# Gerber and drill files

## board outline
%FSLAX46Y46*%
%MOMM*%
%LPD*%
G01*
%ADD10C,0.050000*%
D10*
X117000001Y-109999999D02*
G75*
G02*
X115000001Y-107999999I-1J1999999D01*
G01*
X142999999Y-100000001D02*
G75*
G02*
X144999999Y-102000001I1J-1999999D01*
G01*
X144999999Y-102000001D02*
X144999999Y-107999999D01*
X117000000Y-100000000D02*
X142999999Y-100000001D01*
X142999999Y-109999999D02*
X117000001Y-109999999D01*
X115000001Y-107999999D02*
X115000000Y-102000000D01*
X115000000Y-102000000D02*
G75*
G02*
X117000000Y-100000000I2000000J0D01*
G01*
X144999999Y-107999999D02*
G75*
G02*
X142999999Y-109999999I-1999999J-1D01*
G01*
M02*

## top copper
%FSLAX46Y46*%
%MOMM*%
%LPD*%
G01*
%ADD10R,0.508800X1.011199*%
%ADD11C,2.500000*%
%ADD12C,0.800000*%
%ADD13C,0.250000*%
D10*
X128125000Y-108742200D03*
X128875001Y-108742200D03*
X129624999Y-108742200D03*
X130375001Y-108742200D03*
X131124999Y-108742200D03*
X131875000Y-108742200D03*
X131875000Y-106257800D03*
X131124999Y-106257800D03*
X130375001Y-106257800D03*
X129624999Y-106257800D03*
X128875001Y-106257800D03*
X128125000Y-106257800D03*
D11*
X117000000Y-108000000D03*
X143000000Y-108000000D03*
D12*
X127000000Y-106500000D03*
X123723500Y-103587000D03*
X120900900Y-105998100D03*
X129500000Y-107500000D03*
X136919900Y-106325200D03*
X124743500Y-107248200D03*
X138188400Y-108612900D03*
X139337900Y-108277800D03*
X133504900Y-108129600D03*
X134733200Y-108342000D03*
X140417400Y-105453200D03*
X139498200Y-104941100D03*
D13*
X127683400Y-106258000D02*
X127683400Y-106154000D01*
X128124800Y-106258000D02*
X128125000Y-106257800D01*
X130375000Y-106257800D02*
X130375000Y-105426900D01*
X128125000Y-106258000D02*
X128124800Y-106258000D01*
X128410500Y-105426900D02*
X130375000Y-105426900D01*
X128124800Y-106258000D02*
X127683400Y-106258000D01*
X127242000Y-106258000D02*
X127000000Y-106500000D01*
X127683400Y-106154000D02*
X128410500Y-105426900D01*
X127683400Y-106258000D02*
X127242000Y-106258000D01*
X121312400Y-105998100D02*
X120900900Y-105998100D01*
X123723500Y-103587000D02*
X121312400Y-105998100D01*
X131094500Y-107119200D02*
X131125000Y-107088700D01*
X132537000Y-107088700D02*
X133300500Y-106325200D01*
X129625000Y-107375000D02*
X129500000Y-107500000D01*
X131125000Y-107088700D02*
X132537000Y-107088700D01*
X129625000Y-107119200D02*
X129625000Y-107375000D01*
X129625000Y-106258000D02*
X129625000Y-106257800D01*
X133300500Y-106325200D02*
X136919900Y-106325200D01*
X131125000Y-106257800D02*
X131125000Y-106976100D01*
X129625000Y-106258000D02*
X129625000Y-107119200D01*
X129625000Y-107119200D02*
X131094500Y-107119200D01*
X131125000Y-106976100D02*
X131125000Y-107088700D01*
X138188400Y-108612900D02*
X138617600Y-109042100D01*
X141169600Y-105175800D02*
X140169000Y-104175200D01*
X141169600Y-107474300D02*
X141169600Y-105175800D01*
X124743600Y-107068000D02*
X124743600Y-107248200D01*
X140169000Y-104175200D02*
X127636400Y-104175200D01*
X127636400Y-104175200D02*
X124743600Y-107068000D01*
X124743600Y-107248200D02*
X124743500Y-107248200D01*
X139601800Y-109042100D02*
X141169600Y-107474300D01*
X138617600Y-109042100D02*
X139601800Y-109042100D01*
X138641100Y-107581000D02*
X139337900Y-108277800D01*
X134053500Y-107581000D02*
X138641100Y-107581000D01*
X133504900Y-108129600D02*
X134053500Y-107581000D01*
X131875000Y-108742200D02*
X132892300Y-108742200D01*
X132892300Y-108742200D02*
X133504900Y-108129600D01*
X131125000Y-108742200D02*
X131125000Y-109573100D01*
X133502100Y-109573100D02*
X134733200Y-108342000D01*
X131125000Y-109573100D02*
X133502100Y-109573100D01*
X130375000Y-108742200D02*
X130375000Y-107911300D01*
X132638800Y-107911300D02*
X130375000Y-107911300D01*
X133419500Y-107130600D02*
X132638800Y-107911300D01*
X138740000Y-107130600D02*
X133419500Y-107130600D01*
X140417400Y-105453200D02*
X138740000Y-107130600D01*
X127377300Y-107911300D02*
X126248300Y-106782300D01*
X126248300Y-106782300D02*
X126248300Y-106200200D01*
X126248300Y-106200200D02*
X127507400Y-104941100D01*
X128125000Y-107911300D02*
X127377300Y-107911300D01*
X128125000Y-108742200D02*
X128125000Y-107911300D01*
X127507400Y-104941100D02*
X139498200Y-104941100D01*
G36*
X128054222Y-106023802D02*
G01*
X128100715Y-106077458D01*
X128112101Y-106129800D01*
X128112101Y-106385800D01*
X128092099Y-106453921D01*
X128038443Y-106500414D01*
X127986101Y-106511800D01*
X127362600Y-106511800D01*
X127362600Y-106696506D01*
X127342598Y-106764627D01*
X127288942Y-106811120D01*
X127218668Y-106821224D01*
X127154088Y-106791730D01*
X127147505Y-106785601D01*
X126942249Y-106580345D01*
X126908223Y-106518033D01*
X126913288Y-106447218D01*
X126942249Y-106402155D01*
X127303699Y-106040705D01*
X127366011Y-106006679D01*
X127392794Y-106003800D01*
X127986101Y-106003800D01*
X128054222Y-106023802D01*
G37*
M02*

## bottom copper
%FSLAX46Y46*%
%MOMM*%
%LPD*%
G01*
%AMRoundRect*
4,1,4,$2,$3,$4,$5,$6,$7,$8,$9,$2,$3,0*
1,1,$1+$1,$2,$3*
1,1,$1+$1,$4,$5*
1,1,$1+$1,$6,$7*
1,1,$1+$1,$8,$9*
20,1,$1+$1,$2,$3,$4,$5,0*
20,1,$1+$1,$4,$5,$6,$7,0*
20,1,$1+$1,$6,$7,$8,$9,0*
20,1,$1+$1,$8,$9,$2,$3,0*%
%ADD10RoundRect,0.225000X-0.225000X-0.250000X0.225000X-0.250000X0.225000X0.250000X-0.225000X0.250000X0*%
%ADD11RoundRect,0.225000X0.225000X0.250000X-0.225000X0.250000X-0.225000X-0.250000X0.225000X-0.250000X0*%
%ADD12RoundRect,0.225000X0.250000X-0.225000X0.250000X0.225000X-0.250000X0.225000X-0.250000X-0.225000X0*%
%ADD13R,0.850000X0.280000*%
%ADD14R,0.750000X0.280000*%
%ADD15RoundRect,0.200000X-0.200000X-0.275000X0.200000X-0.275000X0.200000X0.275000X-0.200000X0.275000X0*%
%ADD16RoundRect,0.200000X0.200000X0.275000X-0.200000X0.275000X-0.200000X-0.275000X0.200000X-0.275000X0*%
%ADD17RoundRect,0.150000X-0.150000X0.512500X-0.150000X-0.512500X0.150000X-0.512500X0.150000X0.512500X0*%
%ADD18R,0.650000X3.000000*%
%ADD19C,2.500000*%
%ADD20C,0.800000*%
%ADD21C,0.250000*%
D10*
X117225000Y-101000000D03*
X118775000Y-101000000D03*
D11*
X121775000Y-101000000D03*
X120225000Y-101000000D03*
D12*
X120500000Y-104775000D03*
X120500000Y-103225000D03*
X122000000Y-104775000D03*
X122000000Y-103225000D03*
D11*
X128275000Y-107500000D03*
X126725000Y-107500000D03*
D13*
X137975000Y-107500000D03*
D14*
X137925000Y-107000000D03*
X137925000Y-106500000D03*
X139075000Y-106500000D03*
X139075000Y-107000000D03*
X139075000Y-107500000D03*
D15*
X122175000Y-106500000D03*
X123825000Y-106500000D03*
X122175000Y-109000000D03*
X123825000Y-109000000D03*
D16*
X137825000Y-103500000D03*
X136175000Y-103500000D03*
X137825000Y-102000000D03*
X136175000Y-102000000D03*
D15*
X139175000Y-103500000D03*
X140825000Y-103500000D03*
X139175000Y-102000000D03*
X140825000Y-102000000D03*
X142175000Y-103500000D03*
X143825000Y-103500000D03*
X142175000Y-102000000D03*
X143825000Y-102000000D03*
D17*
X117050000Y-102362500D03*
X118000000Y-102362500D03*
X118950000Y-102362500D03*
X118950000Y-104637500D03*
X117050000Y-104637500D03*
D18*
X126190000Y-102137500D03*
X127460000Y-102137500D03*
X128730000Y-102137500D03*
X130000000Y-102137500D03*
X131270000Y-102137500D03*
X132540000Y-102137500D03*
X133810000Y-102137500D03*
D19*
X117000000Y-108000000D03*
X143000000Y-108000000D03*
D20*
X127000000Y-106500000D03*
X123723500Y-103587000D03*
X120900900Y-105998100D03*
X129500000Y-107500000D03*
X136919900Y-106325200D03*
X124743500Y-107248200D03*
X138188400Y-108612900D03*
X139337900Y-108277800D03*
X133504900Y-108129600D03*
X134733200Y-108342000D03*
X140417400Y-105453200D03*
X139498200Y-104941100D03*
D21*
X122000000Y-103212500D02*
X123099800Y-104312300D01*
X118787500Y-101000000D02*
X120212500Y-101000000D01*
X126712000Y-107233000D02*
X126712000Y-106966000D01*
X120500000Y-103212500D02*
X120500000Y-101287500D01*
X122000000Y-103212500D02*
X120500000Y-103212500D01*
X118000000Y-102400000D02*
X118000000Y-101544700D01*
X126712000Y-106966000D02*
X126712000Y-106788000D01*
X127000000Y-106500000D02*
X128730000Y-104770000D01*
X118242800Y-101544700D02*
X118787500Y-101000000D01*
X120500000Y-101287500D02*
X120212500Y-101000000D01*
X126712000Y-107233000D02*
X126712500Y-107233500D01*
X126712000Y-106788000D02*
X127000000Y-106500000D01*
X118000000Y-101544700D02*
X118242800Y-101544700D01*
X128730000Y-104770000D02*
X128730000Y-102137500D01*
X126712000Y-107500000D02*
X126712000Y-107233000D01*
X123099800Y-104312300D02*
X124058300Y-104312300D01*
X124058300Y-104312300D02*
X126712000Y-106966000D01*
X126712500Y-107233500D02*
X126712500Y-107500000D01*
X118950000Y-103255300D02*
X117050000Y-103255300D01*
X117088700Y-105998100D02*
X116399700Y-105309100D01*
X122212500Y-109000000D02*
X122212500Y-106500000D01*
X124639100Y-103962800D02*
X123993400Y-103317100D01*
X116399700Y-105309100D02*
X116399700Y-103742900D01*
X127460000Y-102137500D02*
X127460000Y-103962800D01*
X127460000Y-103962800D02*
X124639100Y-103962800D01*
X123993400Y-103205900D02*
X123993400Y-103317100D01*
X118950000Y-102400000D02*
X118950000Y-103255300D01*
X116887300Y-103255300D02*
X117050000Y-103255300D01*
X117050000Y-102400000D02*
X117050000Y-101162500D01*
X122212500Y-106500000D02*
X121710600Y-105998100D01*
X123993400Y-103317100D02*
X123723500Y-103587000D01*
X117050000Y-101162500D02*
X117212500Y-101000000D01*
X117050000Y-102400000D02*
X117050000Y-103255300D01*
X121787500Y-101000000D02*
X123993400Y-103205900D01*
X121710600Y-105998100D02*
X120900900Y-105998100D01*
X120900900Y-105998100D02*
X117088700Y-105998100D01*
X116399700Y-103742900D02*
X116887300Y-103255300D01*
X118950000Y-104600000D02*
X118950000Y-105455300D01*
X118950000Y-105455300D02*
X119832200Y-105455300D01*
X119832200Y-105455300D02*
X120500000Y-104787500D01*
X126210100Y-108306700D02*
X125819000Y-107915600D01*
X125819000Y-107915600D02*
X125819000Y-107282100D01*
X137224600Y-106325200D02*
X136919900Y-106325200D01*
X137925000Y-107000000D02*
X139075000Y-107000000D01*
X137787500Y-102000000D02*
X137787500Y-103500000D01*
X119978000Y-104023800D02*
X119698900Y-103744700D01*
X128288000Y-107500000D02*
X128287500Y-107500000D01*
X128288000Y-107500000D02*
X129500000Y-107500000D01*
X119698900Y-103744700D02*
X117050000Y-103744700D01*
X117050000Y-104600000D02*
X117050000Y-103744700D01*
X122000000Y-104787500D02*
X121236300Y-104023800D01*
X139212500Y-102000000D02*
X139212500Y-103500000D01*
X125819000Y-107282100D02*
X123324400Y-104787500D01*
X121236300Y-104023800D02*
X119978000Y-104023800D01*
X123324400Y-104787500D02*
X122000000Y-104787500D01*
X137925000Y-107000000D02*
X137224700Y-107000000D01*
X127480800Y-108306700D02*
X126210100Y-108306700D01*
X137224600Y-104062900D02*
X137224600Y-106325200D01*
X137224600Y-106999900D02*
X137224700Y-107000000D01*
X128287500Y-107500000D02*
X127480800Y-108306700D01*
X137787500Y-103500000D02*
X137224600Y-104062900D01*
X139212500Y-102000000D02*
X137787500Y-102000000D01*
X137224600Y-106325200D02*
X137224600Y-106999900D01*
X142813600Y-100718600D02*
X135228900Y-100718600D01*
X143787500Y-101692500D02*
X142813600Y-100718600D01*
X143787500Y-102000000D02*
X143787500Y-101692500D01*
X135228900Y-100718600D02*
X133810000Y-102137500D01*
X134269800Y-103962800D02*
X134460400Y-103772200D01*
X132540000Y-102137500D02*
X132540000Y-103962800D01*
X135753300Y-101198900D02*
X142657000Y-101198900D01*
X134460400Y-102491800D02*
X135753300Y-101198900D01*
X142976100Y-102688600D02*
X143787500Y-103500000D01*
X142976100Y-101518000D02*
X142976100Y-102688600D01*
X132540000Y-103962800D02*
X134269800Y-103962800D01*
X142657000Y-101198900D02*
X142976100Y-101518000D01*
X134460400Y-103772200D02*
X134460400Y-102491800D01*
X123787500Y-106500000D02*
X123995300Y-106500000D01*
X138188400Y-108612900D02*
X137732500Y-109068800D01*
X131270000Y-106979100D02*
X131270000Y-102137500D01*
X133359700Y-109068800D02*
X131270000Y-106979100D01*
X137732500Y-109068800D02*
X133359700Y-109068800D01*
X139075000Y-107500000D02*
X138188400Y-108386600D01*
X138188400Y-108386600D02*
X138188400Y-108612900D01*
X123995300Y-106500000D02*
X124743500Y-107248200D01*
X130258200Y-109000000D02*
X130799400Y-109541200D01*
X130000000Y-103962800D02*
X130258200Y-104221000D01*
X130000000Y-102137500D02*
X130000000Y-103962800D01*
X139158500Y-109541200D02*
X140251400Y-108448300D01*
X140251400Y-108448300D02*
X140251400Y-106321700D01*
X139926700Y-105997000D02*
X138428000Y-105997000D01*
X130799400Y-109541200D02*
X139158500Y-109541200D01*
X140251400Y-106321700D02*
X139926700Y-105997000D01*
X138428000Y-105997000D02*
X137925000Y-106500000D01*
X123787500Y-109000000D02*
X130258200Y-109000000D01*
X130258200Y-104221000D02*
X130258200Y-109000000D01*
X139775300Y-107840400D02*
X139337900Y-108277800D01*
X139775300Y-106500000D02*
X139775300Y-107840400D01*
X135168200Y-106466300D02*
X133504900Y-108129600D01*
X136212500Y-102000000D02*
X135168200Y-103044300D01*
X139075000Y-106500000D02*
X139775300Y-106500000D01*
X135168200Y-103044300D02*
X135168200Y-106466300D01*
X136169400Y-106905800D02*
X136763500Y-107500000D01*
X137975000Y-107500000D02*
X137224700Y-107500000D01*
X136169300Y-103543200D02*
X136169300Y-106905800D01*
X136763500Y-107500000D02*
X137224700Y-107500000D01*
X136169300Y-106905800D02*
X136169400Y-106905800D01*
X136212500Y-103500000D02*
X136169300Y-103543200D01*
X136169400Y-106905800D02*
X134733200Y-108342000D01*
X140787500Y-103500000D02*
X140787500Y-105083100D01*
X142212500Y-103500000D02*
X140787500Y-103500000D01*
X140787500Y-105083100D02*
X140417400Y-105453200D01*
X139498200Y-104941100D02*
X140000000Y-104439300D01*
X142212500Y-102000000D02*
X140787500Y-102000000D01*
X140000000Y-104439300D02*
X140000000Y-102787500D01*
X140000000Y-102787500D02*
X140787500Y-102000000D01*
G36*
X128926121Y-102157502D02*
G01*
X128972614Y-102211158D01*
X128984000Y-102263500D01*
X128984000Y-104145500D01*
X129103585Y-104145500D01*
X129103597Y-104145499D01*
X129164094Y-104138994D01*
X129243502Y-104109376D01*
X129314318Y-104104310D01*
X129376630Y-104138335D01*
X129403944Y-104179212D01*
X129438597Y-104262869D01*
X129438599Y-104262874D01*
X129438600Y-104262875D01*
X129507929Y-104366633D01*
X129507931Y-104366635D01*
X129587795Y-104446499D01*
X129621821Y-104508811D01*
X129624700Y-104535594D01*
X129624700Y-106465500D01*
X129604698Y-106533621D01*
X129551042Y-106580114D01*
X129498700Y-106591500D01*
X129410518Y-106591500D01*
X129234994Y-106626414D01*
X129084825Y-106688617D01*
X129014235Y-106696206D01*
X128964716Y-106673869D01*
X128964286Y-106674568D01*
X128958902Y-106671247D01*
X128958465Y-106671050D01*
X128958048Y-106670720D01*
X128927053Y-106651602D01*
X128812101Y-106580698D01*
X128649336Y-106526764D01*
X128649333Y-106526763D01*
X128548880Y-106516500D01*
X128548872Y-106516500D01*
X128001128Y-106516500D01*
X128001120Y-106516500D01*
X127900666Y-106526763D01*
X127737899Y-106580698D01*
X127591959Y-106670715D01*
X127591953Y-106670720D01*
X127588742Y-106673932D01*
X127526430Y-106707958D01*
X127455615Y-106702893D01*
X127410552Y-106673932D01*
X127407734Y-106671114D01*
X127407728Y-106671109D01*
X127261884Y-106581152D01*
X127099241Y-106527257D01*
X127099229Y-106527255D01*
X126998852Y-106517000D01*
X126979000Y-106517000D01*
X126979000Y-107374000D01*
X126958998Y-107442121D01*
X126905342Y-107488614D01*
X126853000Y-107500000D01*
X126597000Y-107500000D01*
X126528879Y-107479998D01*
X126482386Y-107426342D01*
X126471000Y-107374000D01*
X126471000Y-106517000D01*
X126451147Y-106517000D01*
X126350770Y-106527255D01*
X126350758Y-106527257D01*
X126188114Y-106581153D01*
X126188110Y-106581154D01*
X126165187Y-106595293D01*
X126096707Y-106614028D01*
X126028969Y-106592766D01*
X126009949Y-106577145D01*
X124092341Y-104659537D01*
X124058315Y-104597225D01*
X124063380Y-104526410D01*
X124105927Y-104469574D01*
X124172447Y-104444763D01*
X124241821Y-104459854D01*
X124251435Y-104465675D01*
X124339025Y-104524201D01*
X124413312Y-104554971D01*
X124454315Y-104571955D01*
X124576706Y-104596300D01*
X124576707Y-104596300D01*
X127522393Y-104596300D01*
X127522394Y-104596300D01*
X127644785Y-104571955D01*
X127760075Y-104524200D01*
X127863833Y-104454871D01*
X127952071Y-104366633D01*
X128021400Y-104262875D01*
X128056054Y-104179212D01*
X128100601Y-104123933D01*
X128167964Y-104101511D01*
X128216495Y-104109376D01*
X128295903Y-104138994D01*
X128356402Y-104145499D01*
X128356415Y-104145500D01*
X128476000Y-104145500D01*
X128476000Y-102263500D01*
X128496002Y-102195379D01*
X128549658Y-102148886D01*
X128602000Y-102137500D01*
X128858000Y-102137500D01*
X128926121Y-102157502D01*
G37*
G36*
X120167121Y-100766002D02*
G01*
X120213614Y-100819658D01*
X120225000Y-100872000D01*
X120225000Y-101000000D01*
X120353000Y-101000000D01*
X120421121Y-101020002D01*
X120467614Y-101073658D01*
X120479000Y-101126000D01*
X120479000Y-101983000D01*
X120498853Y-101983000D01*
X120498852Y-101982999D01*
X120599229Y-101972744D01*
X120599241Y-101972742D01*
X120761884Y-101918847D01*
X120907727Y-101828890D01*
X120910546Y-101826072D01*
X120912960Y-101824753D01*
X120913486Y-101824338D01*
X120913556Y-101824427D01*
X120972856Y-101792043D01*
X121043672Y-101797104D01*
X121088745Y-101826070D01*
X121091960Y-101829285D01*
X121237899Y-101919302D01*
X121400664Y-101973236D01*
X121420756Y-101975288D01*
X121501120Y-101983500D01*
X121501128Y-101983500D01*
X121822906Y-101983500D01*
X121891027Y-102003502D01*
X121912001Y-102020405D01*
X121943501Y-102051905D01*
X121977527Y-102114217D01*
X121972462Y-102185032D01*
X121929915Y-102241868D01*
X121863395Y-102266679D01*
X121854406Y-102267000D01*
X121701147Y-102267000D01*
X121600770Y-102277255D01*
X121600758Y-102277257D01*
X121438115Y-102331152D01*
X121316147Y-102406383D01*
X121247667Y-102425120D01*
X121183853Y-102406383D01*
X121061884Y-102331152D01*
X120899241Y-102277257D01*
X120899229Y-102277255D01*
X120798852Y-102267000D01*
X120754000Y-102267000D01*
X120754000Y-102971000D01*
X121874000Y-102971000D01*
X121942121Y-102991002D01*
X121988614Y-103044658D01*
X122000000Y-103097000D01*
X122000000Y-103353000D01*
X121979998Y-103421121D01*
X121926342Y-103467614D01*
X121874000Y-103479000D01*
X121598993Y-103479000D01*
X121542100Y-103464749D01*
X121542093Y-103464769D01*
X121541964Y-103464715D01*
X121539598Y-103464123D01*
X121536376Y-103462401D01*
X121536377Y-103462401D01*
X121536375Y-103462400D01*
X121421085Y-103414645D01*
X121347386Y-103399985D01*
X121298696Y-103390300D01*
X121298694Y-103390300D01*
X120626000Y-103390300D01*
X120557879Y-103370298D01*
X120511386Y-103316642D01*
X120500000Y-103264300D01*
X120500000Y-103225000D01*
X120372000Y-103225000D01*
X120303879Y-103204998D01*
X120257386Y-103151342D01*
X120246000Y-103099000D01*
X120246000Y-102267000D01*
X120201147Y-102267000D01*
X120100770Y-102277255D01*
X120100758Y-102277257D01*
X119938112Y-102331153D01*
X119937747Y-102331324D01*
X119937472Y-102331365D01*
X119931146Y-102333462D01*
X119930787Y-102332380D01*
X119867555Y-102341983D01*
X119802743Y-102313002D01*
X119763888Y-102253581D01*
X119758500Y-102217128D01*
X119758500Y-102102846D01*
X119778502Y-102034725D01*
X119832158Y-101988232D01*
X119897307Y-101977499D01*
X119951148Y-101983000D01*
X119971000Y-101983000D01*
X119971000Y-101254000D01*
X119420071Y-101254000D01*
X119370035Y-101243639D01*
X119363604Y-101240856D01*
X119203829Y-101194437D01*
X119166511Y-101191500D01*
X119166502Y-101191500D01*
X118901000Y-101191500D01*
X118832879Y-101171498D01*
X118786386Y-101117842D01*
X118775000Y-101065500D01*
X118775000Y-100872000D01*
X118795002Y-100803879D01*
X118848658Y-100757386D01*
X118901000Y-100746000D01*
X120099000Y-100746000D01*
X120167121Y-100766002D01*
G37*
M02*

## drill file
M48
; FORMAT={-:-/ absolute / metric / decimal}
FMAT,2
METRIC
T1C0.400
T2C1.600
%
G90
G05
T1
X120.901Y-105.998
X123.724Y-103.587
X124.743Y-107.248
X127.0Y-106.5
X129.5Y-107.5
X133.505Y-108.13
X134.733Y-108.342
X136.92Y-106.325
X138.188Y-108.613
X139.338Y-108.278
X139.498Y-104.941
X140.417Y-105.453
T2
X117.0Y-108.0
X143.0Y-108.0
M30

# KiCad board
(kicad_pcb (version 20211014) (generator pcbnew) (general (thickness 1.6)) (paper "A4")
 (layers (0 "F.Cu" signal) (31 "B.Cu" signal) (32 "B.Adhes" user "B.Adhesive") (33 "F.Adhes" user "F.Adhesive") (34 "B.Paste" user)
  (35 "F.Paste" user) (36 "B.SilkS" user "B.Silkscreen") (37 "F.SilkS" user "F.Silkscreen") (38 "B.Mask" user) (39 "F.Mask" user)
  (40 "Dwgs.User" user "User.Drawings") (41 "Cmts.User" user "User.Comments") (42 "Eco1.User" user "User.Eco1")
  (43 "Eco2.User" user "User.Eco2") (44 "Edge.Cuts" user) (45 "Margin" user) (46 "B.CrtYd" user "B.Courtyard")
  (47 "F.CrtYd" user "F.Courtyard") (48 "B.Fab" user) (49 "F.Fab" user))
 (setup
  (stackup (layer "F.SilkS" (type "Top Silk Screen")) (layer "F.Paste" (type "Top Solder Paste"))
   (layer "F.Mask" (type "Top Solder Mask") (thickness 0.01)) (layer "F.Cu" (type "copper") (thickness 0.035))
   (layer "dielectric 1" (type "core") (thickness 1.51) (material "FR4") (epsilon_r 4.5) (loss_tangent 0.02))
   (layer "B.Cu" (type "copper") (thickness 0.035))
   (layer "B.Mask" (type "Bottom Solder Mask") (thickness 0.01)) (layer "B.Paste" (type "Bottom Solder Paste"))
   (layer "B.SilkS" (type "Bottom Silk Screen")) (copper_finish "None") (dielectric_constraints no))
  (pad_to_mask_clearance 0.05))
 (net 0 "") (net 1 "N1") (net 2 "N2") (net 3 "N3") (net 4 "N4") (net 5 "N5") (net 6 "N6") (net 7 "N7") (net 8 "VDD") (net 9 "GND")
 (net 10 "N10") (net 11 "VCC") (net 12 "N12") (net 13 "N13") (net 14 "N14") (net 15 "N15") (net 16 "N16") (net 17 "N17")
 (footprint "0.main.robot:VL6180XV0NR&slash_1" (layer "F.Cu") (at 130 107.5 90)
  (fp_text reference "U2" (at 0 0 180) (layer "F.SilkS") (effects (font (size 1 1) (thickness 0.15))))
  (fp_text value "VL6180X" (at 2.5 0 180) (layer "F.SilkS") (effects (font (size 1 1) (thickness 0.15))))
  (pad "1" smd rect (at -1.2422 -1.875 90) (size 1.011199 0.5088) (layers "F.Cu" "F.Paste" "F.Mask") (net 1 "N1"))
  (pad "2" smd rect (at -1.2422 -1.124999 90) (size 1.011199 0.5088) (layers "F.Cu" "F.Paste" "F.Mask") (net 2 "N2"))
  (pad "3" smd rect (at -1.2422 -0.375001 90) (size 1.011199 0.5088) (layers "F.Cu" "F.Paste" "F.Mask") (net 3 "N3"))
  (pad "4" smd rect (at -1.2422 0.375001 90) (size 1.011199 0.5088) (layers "F.Cu" "F.Paste" "F.Mask") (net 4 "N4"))
  (pad "5" smd rect (at -1.2422 1.124999 90) (size 1.011199 0.5088) (layers "F.Cu" "F.Paste" "F.Mask") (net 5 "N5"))
  (pad "6" smd rect (at -1.2422 1.875 90) (size 1.011199 0.5088) (layers "F.Cu" "F.Paste" "F.Mask") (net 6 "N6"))
  (pad "7" smd rect (at 1.2422 1.875 90) (size 1.011199 0.5088) (layers "F.Cu" "F.Paste" "F.Mask") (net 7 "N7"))
  (pad "8" smd rect (at 1.2422 1.124999 90) (size 1.011199 0.5088) (layers "F.Cu" "F.Paste" "F.Mask") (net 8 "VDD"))
  (pad "9" smd rect (at 1.2422 0.375001 90) (size 1.011199 0.5088) (layers "F.Cu" "F.Paste" "F.Mask") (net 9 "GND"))
  (pad "10" smd rect (at 1.2422 -0.375001 90) (size 1.011199 0.5088) (layers "F.Cu" "F.Paste" "F.Mask") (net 8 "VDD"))
  (pad "11" smd rect (at 1.2422 -1.124999 90) (size 1.011199 0.5088) (layers "F.Cu" "F.Paste" "F.Mask") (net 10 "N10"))
  (pad "12" smd rect (at 1.2422 -1.875 90) (size 1.011199 0.5088) (layers "F.Cu" "F.Paste" "F.Mask") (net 9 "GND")))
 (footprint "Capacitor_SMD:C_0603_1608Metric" (layer "B.Cu") (at 118 101)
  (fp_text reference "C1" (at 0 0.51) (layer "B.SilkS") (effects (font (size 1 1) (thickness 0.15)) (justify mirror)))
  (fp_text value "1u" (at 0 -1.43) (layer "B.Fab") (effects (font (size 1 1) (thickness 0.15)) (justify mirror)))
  (pad "1" smd roundrect (at -0.775 0) (size 0.9 0.95) (layers "B.Cu" "B.Paste" "B.Mask") (roundrect_rratio 0.25) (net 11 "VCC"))
  (pad "2" smd roundrect (at 0.775 0) (size 0.9 0.95) (layers "B.Cu" "B.Paste" "B.Mask") (roundrect_rratio 0.25) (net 9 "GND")))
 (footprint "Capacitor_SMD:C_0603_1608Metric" (layer "B.Cu") (at 121 101 180)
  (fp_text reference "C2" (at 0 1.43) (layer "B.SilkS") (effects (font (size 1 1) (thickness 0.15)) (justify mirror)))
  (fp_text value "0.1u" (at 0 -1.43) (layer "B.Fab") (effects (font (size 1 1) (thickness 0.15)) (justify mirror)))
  (pad "1" smd roundrect (at -0.775 0 180) (size 0.9 0.95) (layers "B.Cu" "B.Paste" "B.Mask") (roundrect_rratio 0.25) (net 11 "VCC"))
  (pad "2" smd roundrect (at 0.775 0 180) (size 0.9 0.95) (layers "B.Cu" "B.Paste" "B.Mask") (roundrect_rratio 0.25) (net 9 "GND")))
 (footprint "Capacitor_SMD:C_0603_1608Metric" (layer "B.Cu") (at 120.5 104 90)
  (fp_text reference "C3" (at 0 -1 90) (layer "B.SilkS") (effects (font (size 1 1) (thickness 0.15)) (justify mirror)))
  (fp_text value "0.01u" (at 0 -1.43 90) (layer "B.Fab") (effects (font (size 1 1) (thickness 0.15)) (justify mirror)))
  (pad "1" smd roundrect (at -0.775 0 90) (size 0.9 0.95) (layers "B.Cu" "B.Paste" "B.Mask") (roundrect_rratio 0.25) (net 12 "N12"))
  (pad "2" smd roundrect (at 0.775 0 90) (size 0.9 0.95) (layers "B.Cu" "B.Paste" "B.Mask") (roundrect_rratio 0.25) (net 9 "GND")))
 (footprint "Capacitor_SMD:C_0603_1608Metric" (layer "B.Cu") (at 122 104 90)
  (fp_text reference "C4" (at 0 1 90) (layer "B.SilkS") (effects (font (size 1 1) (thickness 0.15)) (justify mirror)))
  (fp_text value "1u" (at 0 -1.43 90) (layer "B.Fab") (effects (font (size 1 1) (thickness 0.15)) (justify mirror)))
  (pad "1" smd roundrect (at -0.775 0 90) (size 0.9 0.95) (layers "B.Cu" "B.Paste" "B.Mask") (roundrect_rratio 0.25) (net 8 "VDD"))
  (pad "2" smd roundrect (at 0.775 0 90) (size 0.9 0.95) (layers "B.Cu" "B.Paste" "B.Mask") (roundrect_rratio 0.25) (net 9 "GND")))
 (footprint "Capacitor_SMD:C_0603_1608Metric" (layer "B.Cu") (at 127.5 107.5 180)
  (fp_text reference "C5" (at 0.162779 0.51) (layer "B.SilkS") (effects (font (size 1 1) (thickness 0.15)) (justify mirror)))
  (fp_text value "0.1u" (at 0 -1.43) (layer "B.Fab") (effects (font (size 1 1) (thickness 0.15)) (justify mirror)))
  (pad "1" smd roundrect (at -0.775 0 180) (size 0.9 0.95) (layers "B.Cu" "B.Paste" "B.Mask") (roundrect_rratio 0.25) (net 8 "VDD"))
  (pad "2" smd roundrect (at 0.775 0 180) (size 0.9 0.95) (layers "B.Cu" "B.Paste" "B.Mask") (roundrect_rratio 0.25) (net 9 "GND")))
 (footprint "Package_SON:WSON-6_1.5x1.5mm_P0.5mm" (layer "B.Cu") (at 138.5 107)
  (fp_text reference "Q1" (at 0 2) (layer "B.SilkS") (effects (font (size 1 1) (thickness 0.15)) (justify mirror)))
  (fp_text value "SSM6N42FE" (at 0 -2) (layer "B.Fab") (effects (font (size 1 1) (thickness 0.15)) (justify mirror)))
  (pad "1" smd rect (at -0.525 0.5 90) (size 0.28 0.85) (layers "B.Cu" "B.Paste" "B.Mask") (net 5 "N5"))
  (pad "2" smd rect (at -0.575 0 90) (size 0.28 0.75) (layers "B.Cu" "B.Paste" "B.Mask") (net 8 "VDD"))
  (pad "3" smd rect (at -0.575 -0.5 90) (size 0.28 0.75) (layers "B.Cu" "B.Paste" "B.Mask") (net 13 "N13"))
  (pad "4" smd rect (at 0.575 -0.5 90) (size 0.28 0.75) (layers "B.Cu" "B.Paste" "B.Mask") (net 6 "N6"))
  (pad "5" smd rect (at 0.575 0 90) (size 0.28 0.75) (layers "B.Cu" "B.Paste" "B.Mask") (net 8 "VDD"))
  (pad "6" smd rect (at 0.575 0.5 90) (size 0.28 0.75) (layers "B.Cu" "B.Paste" "B.Mask") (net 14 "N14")))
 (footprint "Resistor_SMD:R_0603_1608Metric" (layer "B.Cu") (at 123 106.5)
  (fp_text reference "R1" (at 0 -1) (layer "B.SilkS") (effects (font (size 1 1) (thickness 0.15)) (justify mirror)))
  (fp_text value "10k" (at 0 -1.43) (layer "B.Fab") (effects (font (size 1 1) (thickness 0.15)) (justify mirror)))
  (pad "1" smd roundrect (at -0.825 0) (size 0.8 0.95) (layers "B.Cu" "B.Paste" "B.Mask") (roundrect_rratio 0.25) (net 11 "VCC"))
  (pad "2" smd roundrect (at 0.825 0) (size 0.8 0.95) (layers "B.Cu" "B.Paste" "B.Mask") (roundrect_rratio 0.25) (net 14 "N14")))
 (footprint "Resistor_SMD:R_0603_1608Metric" (layer "B.Cu") (at 123 109)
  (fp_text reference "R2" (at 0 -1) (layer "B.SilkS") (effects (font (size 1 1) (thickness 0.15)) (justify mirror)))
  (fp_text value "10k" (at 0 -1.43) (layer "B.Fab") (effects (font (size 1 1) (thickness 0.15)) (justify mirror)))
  (pad "1" smd roundrect (at -0.825 0) (size 0.8 0.95) (layers "B.Cu" "B.Paste" "B.Mask") (roundrect_rratio 0.25) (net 11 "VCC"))
  (pad "2" smd roundrect (at 0.825 0) (size 0.8 0.95) (layers "B.Cu" "B.Paste" "B.Mask") (roundrect_rratio 0.25) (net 13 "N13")))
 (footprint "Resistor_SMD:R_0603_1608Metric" (layer "B.Cu") (at 137 103.5 180)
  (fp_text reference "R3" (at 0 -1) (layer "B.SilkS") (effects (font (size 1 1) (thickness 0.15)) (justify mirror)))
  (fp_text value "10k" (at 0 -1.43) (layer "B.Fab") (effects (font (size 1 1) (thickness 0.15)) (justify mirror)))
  (pad "1" smd roundrect (at -0.825 0 180) (size 0.8 0.95) (layers "B.Cu" "B.Paste" "B.Mask") (roundrect_rratio 0.25) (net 8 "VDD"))
  (pad "2" smd roundrect (at 0.825 0 180) (size 0.8 0.95) (layers "B.Cu" "B.Paste" "B.Mask") (roundrect_rratio 0.25) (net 5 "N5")))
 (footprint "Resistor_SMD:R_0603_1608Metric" (layer "B.Cu") (at 137 102 180)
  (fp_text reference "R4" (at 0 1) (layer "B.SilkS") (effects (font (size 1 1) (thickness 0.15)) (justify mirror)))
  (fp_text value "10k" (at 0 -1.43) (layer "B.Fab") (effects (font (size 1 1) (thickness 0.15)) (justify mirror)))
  (pad "1" smd roundrect (at -0.825 0 180) (size 0.8 0.95) (layers "B.Cu" "B.Paste" "B.Mask") (roundrect_rratio 0.25) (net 8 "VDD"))
  (pad "2" smd roundrect (at 0.825 0 180) (size 0.8 0.95) (layers "B.Cu" "B.Paste" "B.Mask") (roundrect_rratio 0.25) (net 6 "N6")))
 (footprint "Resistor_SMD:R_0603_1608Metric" (layer "B.Cu") (at 140 103.5)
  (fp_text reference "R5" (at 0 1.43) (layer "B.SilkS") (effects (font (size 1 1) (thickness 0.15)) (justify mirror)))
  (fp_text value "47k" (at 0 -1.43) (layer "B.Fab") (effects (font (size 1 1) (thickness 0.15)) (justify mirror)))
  (pad "1" smd roundrect (at -0.825 0) (size 0.8 0.95) (layers "B.Cu" "B.Paste" "B.Mask") (roundrect_rratio 0.25) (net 8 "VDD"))
  (pad "2" smd roundrect (at 0.825 0) (size 0.8 0.95) (layers "B.Cu" "B.Paste" "B.Mask") (roundrect_rratio 0.25) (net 4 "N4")))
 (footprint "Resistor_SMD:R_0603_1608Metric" (layer "B.Cu") (at 140 102)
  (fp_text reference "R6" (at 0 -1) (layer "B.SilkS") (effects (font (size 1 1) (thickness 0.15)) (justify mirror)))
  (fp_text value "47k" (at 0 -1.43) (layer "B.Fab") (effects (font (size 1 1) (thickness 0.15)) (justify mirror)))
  (pad "1" smd roundrect (at -0.825 0) (size 0.8 0.95) (layers "B.Cu" "B.Paste" "B.Mask") (roundrect_rratio 0.25) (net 8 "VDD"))
  (pad "2" smd roundrect (at 0.825 0) (size 0.8 0.95) (layers "B.Cu" "B.Paste" "B.Mask") (roundrect_rratio 0.25) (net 1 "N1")))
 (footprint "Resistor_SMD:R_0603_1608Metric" (layer "B.Cu") (at 143 103.5)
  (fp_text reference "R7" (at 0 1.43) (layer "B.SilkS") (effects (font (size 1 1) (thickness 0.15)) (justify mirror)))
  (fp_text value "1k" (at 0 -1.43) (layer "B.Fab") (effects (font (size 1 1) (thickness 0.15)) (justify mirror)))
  (pad "1" smd roundrect (at -0.825 0) (size 0.8 0.95) (layers "B.Cu" "B.Paste" "B.Mask") (roundrect_rratio 0.25) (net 4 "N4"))
  (pad "2" smd roundrect (at 0.825 0) (size 0.8 0.95) (layers "B.Cu" "B.Paste" "B.Mask") (roundrect_rratio 0.25) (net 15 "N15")))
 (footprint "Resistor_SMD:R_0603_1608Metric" (layer "B.Cu") (at 143 102)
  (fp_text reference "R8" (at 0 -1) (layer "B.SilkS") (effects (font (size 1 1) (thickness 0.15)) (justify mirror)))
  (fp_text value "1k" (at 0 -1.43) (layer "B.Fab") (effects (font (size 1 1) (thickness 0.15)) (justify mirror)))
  (pad "1" smd roundrect (at -0.825 0) (size 0.8 0.95) (layers "B.Cu" "B.Paste" "B.Mask") (roundrect_rratio 0.25) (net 1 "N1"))
  (pad "2" smd roundrect (at 0.825 0) (size 0.8 0.95) (layers "B.Cu" "B.Paste" "B.Mask") (roundrect_rratio 0.25) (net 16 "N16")))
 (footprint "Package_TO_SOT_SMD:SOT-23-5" (layer "B.Cu") (at 118 103.5 -90)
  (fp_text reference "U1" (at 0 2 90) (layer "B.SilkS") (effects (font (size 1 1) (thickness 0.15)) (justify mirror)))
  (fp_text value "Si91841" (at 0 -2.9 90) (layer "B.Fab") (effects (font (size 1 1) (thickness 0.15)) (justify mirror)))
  (pad "1" smd roundrect (at -1.1375 0.95 270) (size 1.325 0.6) (layers "B.Cu" "B.Paste" "B.Mask") (roundrect_rratio 0.25) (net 11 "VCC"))
  (pad "2" smd roundrect (at -1.1375 0 270) (size 1.325 0.6) (layers "B.Cu" "B.Paste" "B.Mask") (roundrect_rratio 0.25) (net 9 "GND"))
  (pad "3" smd roundrect (at -1.1375 -0.95 270) (size 1.325 0.6) (layers "B.Cu" "B.Paste" "B.Mask") (roundrect_rratio 0.25) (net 11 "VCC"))
  (pad "4" smd roundrect (at 1.1375 -0.95 270) (size 1.325 0.6) (layers "B.Cu" "B.Paste" "B.Mask") (roundrect_rratio 0.25) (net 12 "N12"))
  (pad "5" smd roundrect (at 1.1375 0.95 270) (size 1.325 0.6) (layers "B.Cu" "B.Paste" "B.Mask") (roundrect_rratio 0.25) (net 8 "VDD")))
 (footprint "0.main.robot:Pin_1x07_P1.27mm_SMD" (layer "B.Cu") (at 130 103.6375 -90)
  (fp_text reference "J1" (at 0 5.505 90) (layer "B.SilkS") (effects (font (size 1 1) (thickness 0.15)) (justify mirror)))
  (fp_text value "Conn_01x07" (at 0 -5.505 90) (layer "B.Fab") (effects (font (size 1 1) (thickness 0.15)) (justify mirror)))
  (pad "1" smd rect (at -1.5 3.81 270) (size 3 0.65) (layers "B.Cu" "B.Paste" "B.Mask") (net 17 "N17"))
  (pad "2" smd rect (at -1.5 2.54 270) (size 3 0.65) (layers "B.Cu" "B.Paste" "B.Mask") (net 11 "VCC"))
  (pad "3" smd rect (at -1.5 1.27 270) (size 3 0.65) (layers "B.Cu" "B.Paste" "B.Mask") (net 9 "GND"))
  (pad "4" smd rect (at -1.5 0 270) (size 3 0.65) (layers "B.Cu" "B.Paste" "B.Mask") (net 13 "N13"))
  (pad "5" smd rect (at -1.5 -1.27 270) (size 3 0.65) (layers "B.Cu" "B.Paste" "B.Mask") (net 14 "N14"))
  (pad "6" smd rect (at -1.5 -2.54 270) (size 3 0.65) (layers "B.Cu" "B.Paste" "B.Mask") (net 15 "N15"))
  (pad "7" smd rect (at -1.5 -3.81 270) (size 3 0.65) (layers "B.Cu" "B.Paste" "B.Mask") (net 16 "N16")))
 (gr_arc (start 117.000001 109.999999) (mid 115.585787 109.414213) (end 115.000001 107.999999) (layer "Edge.Cuts") (width 0.05))
 (gr_arc (start 142.999999 100.000001) (mid 144.414213 100.585787) (end 144.999999 102.000001) (layer "Edge.Cuts") (width 0.05))
 (gr_line (start 144.999999 102.000001) (end 144.999999 107.999999) (layer "Edge.Cuts") (width 0.05))
 (gr_line (start 117 100) (end 142.999999 100.000001) (layer "Edge.Cuts") (width 0.05))
 (gr_line (start 142.999999 109.999999) (end 117.000001 109.999999) (layer "Edge.Cuts") (width 0.05))
 (gr_line (start 115.000001 107.999999) (end 115 102) (layer "Edge.Cuts") (width 0.05))
 (gr_arc (start 115 102) (mid 115.585786 100.585786) (end 117 100) (layer "Edge.Cuts") (width 0.05))
 (gr_arc (start 144.999999 107.999999) (mid 144.414213 109.414213) (end 142.999999 109.999999) (layer "Edge.Cuts") (width 0.05))
 (via (at 117 108) (size 2.5) (drill 1.6) (layers "F.Cu" "B.Cu") (free) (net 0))
 (via (at 143 108) (size 2.5) (drill 1.6) (layers "F.Cu" "B.Cu") (free) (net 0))
 (segment (start 127.6834 106.258) (end 127.6834 106.154) (width 0.25) (layer "F.Cu") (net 9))
 (segment (start 128.1248 106.258) (end 128.125 106.2578) (width 0.25) (layer "F.Cu") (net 9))
 (segment (start 130.375 106.2578) (end 130.375 105.4269) (width 0.25) (layer "F.Cu") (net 9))
 (segment (start 128.125 106.258) (end 128.1248 106.258) (width 0.25) (layer "F.Cu") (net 9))
 (segment (start 128.4105 105.4269) (end 130.375 105.4269) (width 0.25) (layer "F.Cu") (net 9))
 (segment (start 128.1248 106.258) (end 127.6834 106.258) (width 0.25) (layer "F.Cu") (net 9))
 (segment (start 127.242 106.258) (end 127 106.5) (width 0.25) (layer "F.Cu") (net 9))
 (segment (start 127.6834 106.154) (end 128.4105 105.4269) (width 0.25) (layer "F.Cu") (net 9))
 (segment (start 127.6834 106.258) (end 127.242 106.258) (width 0.25) (layer "F.Cu") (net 9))
 (via (at 127 106.5) (size 0.8) (drill 0.4) (layers "F.Cu" "B.Cu") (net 9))
 (segment (start 122 103.2125) (end 123.0998 104.3123) (width 0.25) (layer "B.Cu") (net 9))
 (segment (start 118.7875 101) (end 120.2125 101) (width 0.25) (layer "B.Cu") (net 9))
 (segment (start 126.712 107.233) (end 126.712 106.966) (width 0.25) (layer "B.Cu") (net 9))
 (segment (start 120.5 103.2125) (end 120.5 101.2875) (width 0.25) (layer "B.Cu") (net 9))
 (segment (start 122 103.2125) (end 120.5 103.2125) (width 0.25) (layer "B.Cu") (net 9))
 (segment (start 118 102.4) (end 118 101.5447) (width 0.25) (layer "B.Cu") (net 9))
 (segment (start 126.712 106.966) (end 126.712 106.788) (width 0.25) (layer "B.Cu") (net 9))
 (segment (start 127 106.5) (end 128.73 104.77) (width 0.25) (layer "B.Cu") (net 9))
 (segment (start 118.2428 101.5447) (end 118.7875 101) (width 0.25) (layer "B.Cu") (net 9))
 (segment (start 120.5 101.2875) (end 120.2125 101) (width 0.25) (layer "B.Cu") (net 9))
 (segment (start 126.712 107.233) (end 126.7125 107.2335) (width 0.25) (layer "B.Cu") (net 9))
 (segment (start 126.712 106.788) (end 127 106.5) (width 0.25) (layer "B.Cu") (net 9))
 (segment (start 118 101.5447) (end 118.2428 101.5447) (width 0.25) (layer "B.Cu") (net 9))
 (segment (start 128.73 104.77) (end 128.73 102.1375) (width 0.25) (layer "B.Cu") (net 9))
 (segment (start 126.712 107.5) (end 126.712 107.233) (width 0.25) (layer "B.Cu") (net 9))
 (segment (start 123.0998 104.3123) (end 124.0583 104.3123) (width 0.25) (layer "B.Cu") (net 9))
 (segment (start 124.0583 104.3123) (end 126.712 106.966) (width 0.25) (layer "B.Cu") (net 9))
 (segment (start 126.7125 107.2335) (end 126.7125 107.5) (width 0.25) (layer "B.Cu") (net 9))
 (segment (start 121.3124 105.9981) (end 120.9009 105.9981) (width 0.25) (layer "F.Cu") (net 11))
 (segment (start 123.7235 103.587) (end 121.3124 105.9981) (width 0.25) (layer "F.Cu") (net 11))
 (via (at 123.7235 103.587) (size 0.8) (drill 0.4) (layers "F.Cu" "B.Cu") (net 11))
 (via (at 120.9009 105.9981) (size 0.8) (drill 0.4) (layers "F.Cu" "B.Cu") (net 11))
 (segment (start 118.95 103.2553) (end 117.05 103.2553) (width 0.25) (layer "B.Cu") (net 11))
 (segment (start 117.0887 105.9981) (end 116.3997 105.3091) (width 0.25) (layer "B.Cu") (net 11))
 (segment (start 122.2125 109) (end 122.2125 106.5) (width 0.25) (layer "B.Cu") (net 11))
 (segment (start 124.6391 103.9628) (end 123.9934 103.3171) (width 0.25) (layer "B.Cu") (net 11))
 (segment (start 116.3997 105.3091) (end 116.3997 103.7429) (width 0.25) (layer "B.Cu") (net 11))
 (segment (start 127.46 102.1375) (end 127.46 103.9628) (width 0.25) (layer "B.Cu") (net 11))
 (segment (start 127.46 103.9628) (end 124.6391 103.9628) (width 0.25) (layer "B.Cu") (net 11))
 (segment (start 123.9934 103.2059) (end 123.9934 103.3171) (width 0.25) (layer "B.Cu") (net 11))
 (segment (start 118.95 102.4) (end 118.95 103.2553) (width 0.25) (layer "B.Cu") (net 11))
 (segment (start 116.8873 103.2553) (end 117.05 103.2553) (width 0.25) (layer "B.Cu") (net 11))
 (segment (start 117.05 102.4) (end 117.05 101.1625) (width 0.25) (layer "B.Cu") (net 11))
 (segment (start 122.2125 106.5) (end 121.7106 105.9981) (width 0.25) (layer "B.Cu") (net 11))
 (segment (start 123.9934 103.3171) (end 123.7235 103.587) (width 0.25) (layer "B.Cu") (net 11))
 (segment (start 117.05 101.1625) (end 117.2125 101) (width 0.25) (layer "B.Cu") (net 11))
 (segment (start 117.05 102.4) (end 117.05 103.2553) (width 0.25) (layer "B.Cu") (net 11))
 (segment (start 121.7875 101) (end 123.9934 103.2059) (width 0.25) (layer "B.Cu") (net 11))
 (segment (start 121.7106 105.9981) (end 120.9009 105.9981) (width 0.25) (layer "B.Cu") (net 11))
 (segment (start 120.9009 105.9981) (end 117.0887 105.9981) (width 0.25) (layer "B.Cu") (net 11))
 (segment (start 116.3997 103.7429) (end 116.8873 103.2553) (width 0.25) (layer "B.Cu") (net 11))
 (segment (start 118.95 104.6) (end 118.95 105.4553) (width 0.25) (layer "B.Cu") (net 12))
 (segment (start 118.95 105.4553) (end 119.8322 105.4553) (width 0.25) (layer "B.Cu") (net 12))
 (segment (start 119.8322 105.4553) (end 120.5 104.7875) (width 0.25) (layer "B.Cu") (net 12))
 (segment (start 131.0945 107.1192) (end 131.125 107.0887) (width 0.25) (layer "F.Cu") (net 8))
 (segment (start 132.537 107.0887) (end 133.3005 106.3252) (width 0.25) (layer "F.Cu") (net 8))
 (segment (start 129.625 107.375) (end 129.5 107.5) (width 0.25) (layer "F.Cu") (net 8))
 (segment (start 131.125 107.0887) (end 132.537 107.0887) (width 0.25) (layer "F.Cu") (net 8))
 (segment (start 129.625 107.1192) (end 129.625 107.375) (width 0.25) (layer "F.Cu") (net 8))
 (segment (start 129.625 106.258) (end 129.625 106.2578) (width 0.25) (layer "F.Cu") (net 8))
 (segment (start 133.3005 106.3252) (end 136.9199 106.3252) (width 0.25) (layer "F.Cu") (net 8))
 (segment (start 131.125 106.2578) (end 131.125 106.9761) (width 0.25) (layer "F.Cu") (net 8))
 (segment (start 129.625 106.258) (end 129.625 107.1192) (width 0.25) (layer "F.Cu") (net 8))
 (segment (start 129.625 107.1192) (end 131.0945 107.1192) (width 0.25) (layer "F.Cu") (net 8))
 (segment (start 131.125 106.9761) (end 131.125 107.0887) (width 0.25) (layer "F.Cu") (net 8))
 (via (at 129.5 107.5) (size 0.8) (drill 0.4) (layers "F.Cu" "B.Cu") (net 8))
 (via (at 136.9199 106.3252) (size 0.8) (drill 0.4) (layers "F.Cu" "B.Cu") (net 8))
 (segment (start 126.2101 108.3067) (end 125.819 107.9156) (width 0.25) (layer "B.Cu") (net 8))
 (segment (start 125.819 107.9156) (end 125.819 107.2821) (width 0.25) (layer "B.Cu") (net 8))
 (segment (start 137.2246 106.3252) (end 136.9199 106.3252) (width 0.25) (layer "B.Cu") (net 8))
 (segment (start 137.925 107) (end 139.075 107) (width 0.25) (layer "B.Cu") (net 8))
 (segment (start 137.7875 102) (end 137.7875 103.5) (width 0.25) (layer "B.Cu") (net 8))
 (segment (start 119.978 104.0238) (end 119.6989 103.7447) (width 0.25) (layer "B.Cu") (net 8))
 (segment (start 128.288 107.5) (end 128.2875 107.5) (width 0.25) (layer "B.Cu") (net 8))
 (segment (start 128.288 107.5) (end 129.5 107.5) (width 0.25) (layer "B.Cu") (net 8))
 (segment (start 119.6989 103.7447) (end 117.05 103.7447) (width 0.25) (layer "B.Cu") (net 8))
 (segment (start 117.05 104.6) (end 117.05 103.7447) (width 0.25) (layer "B.Cu") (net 8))
 (segment (start 122 104.7875) (end 121.2363 104.0238) (width 0.25) (layer "B.Cu") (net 8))
 (segment (start 139.2125 102) (end 139.2125 103.5) (width 0.25) (layer "B.Cu") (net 8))
 (segment (start 125.819 107.2821) (end 123.3244 104.7875) (width 0.25) (layer "B.Cu") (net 8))
 (segment (start 121.2363 104.0238) (end 119.978 104.0238) (width 0.25) (layer "B.Cu") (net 8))
 (segment (start 123.3244 104.7875) (end 122 104.7875) (width 0.25) (layer "B.Cu") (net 8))
 (segment (start 137.925 107) (end 137.2247 107) (width 0.25) (layer "B.Cu") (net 8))
 (segment (start 127.4808 108.3067) (end 126.2101 108.3067) (width 0.25) (layer "B.Cu") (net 8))
 (segment (start 137.2246 104.0629) (end 137.2246 106.3252) (width 0.25) (layer "B.Cu") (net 8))
 (segment (start 137.2246 106.9999) (end 137.2247 107) (width 0.25) (layer "B.Cu") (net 8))
 (segment (start 128.2875 107.5) (end 127.4808 108.3067) (width 0.25) (layer "B.Cu") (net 8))
 (segment (start 137.7875 103.5) (end 137.2246 104.0629) (width 0.25) (layer "B.Cu") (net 8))
 (segment (start 139.2125 102) (end 137.7875 102) (width 0.25) (layer "B.Cu") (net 8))
 (segment (start 137.2246 106.3252) (end 137.2246 106.9999) (width 0.25) (layer "B.Cu") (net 8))
 (segment (start 142.8136 100.7186) (end 135.2289 100.7186) (width 0.25) (layer "B.Cu") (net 16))
 (segment (start 143.7875 101.6925) (end 142.8136 100.7186) (width 0.25) (layer "B.Cu") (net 16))
 (segment (start 143.7875 102) (end 143.7875 101.6925) (width 0.25) (layer "B.Cu") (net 16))
 (segment (start 135.2289 100.7186) (end 133.81 102.1375) (width 0.25) (layer "B.Cu") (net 16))
 (segment (start 134.2698 103.9628) (end 134.4604 103.7722) (width 0.25) (layer "B.Cu") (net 15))
 (segment (start 132.54 102.1375) (end 132.54 103.9628) (width 0.25) (layer "B.Cu") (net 15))
 (segment (start 135.7533 101.1989) (end 142.657 101.1989) (width 0.25) (layer "B.Cu") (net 15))
 (segment (start 134.4604 102.4918) (end 135.7533 101.1989) (width 0.25) (layer "B.Cu") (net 15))
 (segment (start 142.9761 102.6886) (end 143.7875 103.5) (width 0.25) (layer "B.Cu") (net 15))
 (segment (start 142.9761 101.518) (end 142.9761 102.6886) (width 0.25) (layer "B.Cu") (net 15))
 (segment (start 132.54 103.9628) (end 134.2698 103.9628) (width 0.25) (layer "B.Cu") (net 15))
 (segment (start 142.657 101.1989) (end 142.9761 101.518) (width 0.25) (layer "B.Cu") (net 15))
 (segment (start 134.4604 103.7722) (end 134.4604 102.4918) (width 0.25) (layer "B.Cu") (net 15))
 (segment (start 138.1884 108.6129) (end 138.6176 109.0421) (width 0.25) (layer "F.Cu") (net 14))
 (segment (start 141.1696 105.1758) (end 140.169 104.1752) (width 0.25) (layer "F.Cu") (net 14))
 (segment (start 141.1696 107.4743) (end 141.1696 105.1758) (width 0.25) (layer "F.Cu") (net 14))
 (segment (start 124.7436 107.068) (end 124.7436 107.2482) (width 0.25) (layer "F.Cu") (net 14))
 (segment (start 140.169 104.1752) (end 127.6364 104.1752) (width 0.25) (layer "F.Cu") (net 14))
 (segment (start 127.6364 104.1752) (end 124.7436 107.068) (width 0.25) (layer "F.Cu") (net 14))
 (segment (start 124.7436 107.2482) (end 124.7435 107.2482) (width 0.25) (layer "F.Cu") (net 14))
 (segment (start 139.6018 109.0421) (end 141.1696 107.4743) (width 0.25) (layer "F.Cu") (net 14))
 (segment (start 138.6176 109.0421) (end 139.6018 109.0421) (width 0.25) (layer "F.Cu") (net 14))
 (via (at 124.7435 107.2482) (size 0.8) (drill 0.4) (layers "F.Cu" "B.Cu") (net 14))
 (via (at 138.1884 108.6129) (size 0.8) (drill 0.4) (layers "F.Cu" "B.Cu") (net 14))
 (segment (start 123.7875 106.5) (end 123.9953 106.5) (width 0.25) (layer "B.Cu") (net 14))
 (segment (start 138.1884 108.6129) (end 137.7325 109.0688) (width 0.25) (layer "B.Cu") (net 14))
 (segment (start 131.27 106.9791) (end 131.27 102.1375) (width 0.25) (layer "B.Cu") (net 14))
 (segment (start 133.3597 109.0688) (end 131.27 106.9791) (width 0.25) (layer "B.Cu") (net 14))
 (segment (start 137.7325 109.0688) (end 133.3597 109.0688) (width 0.25) (layer "B.Cu") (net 14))
 (segment (start 139.075 107.5) (end 138.1884 108.3866) (width 0.25) (layer "B.Cu") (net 14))
 (segment (start 138.1884 108.3866) (end 138.1884 108.6129) (width 0.25) (layer "B.Cu") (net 14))
 (segment (start 123.9953 106.5) (end 124.7435 107.2482) (width 0.25) (layer "B.Cu") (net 14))
 (segment (start 130.2582 109) (end 130.7994 109.5412) (width 0.25) (layer "B.Cu") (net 13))
 (segment (start 130 103.9628) (end 130.2582 104.221) (width 0.25) (layer "B.Cu") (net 13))
 (segment (start 130 102.1375) (end 130 103.9628) (width 0.25) (layer "B.Cu") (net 13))
 (segment (start 139.1585 109.5412) (end 140.2514 108.4483) (width 0.25) (layer "B.Cu") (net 13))
 (segment (start 140.2514 108.4483) (end 140.2514 106.3217) (width 0.25) (layer "B.Cu") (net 13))
 (segment (start 139.9267 105.997) (end 138.428 105.997) (width 0.25) (layer "B.Cu") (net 13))
 (segment (start 130.7994 109.5412) (end 139.1585 109.5412) (width 0.25) (layer "B.Cu") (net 13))
 (segment (start 140.2514 106.3217) (end 139.9267 105.997) (width 0.25) (layer "B.Cu") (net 13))
 (segment (start 138.428 105.997) (end 137.925 106.5) (width 0.25) (layer "B.Cu") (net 13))
 (segment (start 123.7875 109) (end 130.2582 109) (width 0.25) (layer "B.Cu") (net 13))
 (segment (start 130.2582 104.221) (end 130.2582 109) (width 0.25) (layer "B.Cu") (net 13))
 (segment (start 138.6411 107.581) (end 139.3379 108.2778) (width 0.25) (layer "F.Cu") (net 6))
 (segment (start 134.0535 107.581) (end 138.6411 107.581) (width 0.25) (layer "F.Cu") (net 6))
 (segment (start 133.5049 108.1296) (end 134.0535 107.581) (width 0.25) (layer "F.Cu") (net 6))
 (segment (start 131.875 108.7422) (end 132.8923 108.7422) (width 0.25) (layer "F.Cu") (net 6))
 (segment (start 132.8923 108.7422) (end 133.5049 108.1296) (width 0.25) (layer "F.Cu") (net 6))
 (via (at 139.3379 108.2778) (size 0.8) (drill 0.4) (layers "F.Cu" "B.Cu") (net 6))
 (via (at 133.5049 108.1296) (size 0.8) (drill 0.4) (layers "F.Cu" "B.Cu") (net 6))
 (segment (start 139.7753 107.8404) (end 139.3379 108.2778) (width 0.25) (layer "B.Cu") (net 6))
 (segment (start 139.7753 106.5) (end 139.7753 107.8404) (width 0.25) (layer "B.Cu") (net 6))
 (segment (start 135.1682 106.4663) (end 133.5049 108.1296) (width 0.25) (layer "B.Cu") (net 6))
 (segment (start 136.2125 102) (end 135.1682 103.0443) (width 0.25) (layer "B.Cu") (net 6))
 (segment (start 139.075 106.5) (end 139.7753 106.5) (width 0.25) (layer "B.Cu") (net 6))
 (segment (start 135.1682 103.0443) (end 135.1682 106.4663) (width 0.25) (layer "B.Cu") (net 6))
 (segment (start 131.125 108.7422) (end 131.125 109.5731) (width 0.25) (layer "F.Cu") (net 5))
 (segment (start 133.5021 109.5731) (end 134.7332 108.342) (width 0.25) (layer "F.Cu") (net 5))
 (segment (start 131.125 109.5731) (end 133.5021 109.5731) (width 0.25) (layer "F.Cu") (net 5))
 (via (at 134.7332 108.342) (size 0.8) (drill 0.4) (layers "F.Cu" "B.Cu") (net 5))
 (segment (start 136.1694 106.9058) (end 136.7635 107.5) (width 0.25) (layer "B.Cu") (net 5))
 (segment (start 137.975 107.5) (end 137.2247 107.5) (width 0.25) (layer "B.Cu") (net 5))
 (segment (start 136.1693 103.5432) (end 136.1693 106.9058) (width 0.25) (layer "B.Cu") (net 5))
 (segment (start 136.7635 107.5) (end 137.2247 107.5) (width 0.25) (layer "B.Cu") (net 5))
 (segment (start 136.1693 106.9058) (end 136.1694 106.9058) (width 0.25) (layer "B.Cu") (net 5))
 (segment (start 136.2125 103.5) (end 136.1693 103.5432) (width 0.25) (layer "B.Cu") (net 5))
 (segment (start 136.1694 106.9058) (end 134.7332 108.342) (width 0.25) (layer "B.Cu") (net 5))
 (segment (start 130.375 108.7422) (end 130.375 107.9113) (width 0.25) (layer "F.Cu") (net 4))
 (segment (start 132.6388 107.9113) (end 130.375 107.9113) (width 0.25) (layer "F.Cu") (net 4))
 (segment (start 133.4195 107.1306) (end 132.6388 107.9113) (width 0.25) (layer "F.Cu") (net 4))
 (segment (start 138.74 107.1306) (end 133.4195 107.1306) (width 0.25) (layer "F.Cu") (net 4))
 (segment (start 140.4174 105.4532) (end 138.74 107.1306) (width 0.25) (layer "F.Cu") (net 4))
 (via (at 140.4174 105.4532) (size 0.8) (drill 0.4) (layers "F.Cu" "B.Cu") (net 4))
 (segment (start 140.7875 103.5) (end 140.7875 105.0831) (width 0.25) (layer "B.Cu") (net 4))
 (segment (start 142.2125 103.5) (end 140.7875 103.5) (width 0.25) (layer "B.Cu") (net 4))
 (segment (start 140.7875 105.0831) (end 140.4174 105.4532) (width 0.25) (layer "B.Cu") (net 4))
 (segment (start 127.3773 107.9113) (end 126.2483 106.7823) (width 0.25) (layer "F.Cu") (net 1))
 (segment (start 126.2483 106.7823) (end 126.2483 106.2002) (width 0.25) (layer "F.Cu") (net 1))
 (segment (start 126.2483 106.2002) (end 127.5074 104.9411) (width 0.25) (layer "F.Cu") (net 1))
 (segment (start 128.125 107.9113) (end 127.3773 107.9113) (width 0.25) (layer "F.Cu") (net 1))
 (segment (start 128.125 108.7422) (end 128.125 107.9113) (width 0.25) (layer "F.Cu") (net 1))
 (segment (start 127.5074 104.9411) (end 139.4982 104.9411) (width 0.25) (layer "F.Cu") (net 1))
 (via (at 139.4982 104.9411) (size 0.8) (drill 0.4) (layers "F.Cu" "B.Cu") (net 1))
 (segment (start 139.4982 104.9411) (end 140 104.4393) (width 0.25) (layer "B.Cu") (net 1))
 (segment (start 142.2125 102) (end 140.7875 102) (width 0.25) (layer "B.Cu") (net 1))
 (segment (start 140 104.4393) (end 140 102.7875) (width 0.25) (layer "B.Cu") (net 1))
 (segment (start 140 102.7875) (end 140.7875 102) (width 0.25) (layer "B.Cu") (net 1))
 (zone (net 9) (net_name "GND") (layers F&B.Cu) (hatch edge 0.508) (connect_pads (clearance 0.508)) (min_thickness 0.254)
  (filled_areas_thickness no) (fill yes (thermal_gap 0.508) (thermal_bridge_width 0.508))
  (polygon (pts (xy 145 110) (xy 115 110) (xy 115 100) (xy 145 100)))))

